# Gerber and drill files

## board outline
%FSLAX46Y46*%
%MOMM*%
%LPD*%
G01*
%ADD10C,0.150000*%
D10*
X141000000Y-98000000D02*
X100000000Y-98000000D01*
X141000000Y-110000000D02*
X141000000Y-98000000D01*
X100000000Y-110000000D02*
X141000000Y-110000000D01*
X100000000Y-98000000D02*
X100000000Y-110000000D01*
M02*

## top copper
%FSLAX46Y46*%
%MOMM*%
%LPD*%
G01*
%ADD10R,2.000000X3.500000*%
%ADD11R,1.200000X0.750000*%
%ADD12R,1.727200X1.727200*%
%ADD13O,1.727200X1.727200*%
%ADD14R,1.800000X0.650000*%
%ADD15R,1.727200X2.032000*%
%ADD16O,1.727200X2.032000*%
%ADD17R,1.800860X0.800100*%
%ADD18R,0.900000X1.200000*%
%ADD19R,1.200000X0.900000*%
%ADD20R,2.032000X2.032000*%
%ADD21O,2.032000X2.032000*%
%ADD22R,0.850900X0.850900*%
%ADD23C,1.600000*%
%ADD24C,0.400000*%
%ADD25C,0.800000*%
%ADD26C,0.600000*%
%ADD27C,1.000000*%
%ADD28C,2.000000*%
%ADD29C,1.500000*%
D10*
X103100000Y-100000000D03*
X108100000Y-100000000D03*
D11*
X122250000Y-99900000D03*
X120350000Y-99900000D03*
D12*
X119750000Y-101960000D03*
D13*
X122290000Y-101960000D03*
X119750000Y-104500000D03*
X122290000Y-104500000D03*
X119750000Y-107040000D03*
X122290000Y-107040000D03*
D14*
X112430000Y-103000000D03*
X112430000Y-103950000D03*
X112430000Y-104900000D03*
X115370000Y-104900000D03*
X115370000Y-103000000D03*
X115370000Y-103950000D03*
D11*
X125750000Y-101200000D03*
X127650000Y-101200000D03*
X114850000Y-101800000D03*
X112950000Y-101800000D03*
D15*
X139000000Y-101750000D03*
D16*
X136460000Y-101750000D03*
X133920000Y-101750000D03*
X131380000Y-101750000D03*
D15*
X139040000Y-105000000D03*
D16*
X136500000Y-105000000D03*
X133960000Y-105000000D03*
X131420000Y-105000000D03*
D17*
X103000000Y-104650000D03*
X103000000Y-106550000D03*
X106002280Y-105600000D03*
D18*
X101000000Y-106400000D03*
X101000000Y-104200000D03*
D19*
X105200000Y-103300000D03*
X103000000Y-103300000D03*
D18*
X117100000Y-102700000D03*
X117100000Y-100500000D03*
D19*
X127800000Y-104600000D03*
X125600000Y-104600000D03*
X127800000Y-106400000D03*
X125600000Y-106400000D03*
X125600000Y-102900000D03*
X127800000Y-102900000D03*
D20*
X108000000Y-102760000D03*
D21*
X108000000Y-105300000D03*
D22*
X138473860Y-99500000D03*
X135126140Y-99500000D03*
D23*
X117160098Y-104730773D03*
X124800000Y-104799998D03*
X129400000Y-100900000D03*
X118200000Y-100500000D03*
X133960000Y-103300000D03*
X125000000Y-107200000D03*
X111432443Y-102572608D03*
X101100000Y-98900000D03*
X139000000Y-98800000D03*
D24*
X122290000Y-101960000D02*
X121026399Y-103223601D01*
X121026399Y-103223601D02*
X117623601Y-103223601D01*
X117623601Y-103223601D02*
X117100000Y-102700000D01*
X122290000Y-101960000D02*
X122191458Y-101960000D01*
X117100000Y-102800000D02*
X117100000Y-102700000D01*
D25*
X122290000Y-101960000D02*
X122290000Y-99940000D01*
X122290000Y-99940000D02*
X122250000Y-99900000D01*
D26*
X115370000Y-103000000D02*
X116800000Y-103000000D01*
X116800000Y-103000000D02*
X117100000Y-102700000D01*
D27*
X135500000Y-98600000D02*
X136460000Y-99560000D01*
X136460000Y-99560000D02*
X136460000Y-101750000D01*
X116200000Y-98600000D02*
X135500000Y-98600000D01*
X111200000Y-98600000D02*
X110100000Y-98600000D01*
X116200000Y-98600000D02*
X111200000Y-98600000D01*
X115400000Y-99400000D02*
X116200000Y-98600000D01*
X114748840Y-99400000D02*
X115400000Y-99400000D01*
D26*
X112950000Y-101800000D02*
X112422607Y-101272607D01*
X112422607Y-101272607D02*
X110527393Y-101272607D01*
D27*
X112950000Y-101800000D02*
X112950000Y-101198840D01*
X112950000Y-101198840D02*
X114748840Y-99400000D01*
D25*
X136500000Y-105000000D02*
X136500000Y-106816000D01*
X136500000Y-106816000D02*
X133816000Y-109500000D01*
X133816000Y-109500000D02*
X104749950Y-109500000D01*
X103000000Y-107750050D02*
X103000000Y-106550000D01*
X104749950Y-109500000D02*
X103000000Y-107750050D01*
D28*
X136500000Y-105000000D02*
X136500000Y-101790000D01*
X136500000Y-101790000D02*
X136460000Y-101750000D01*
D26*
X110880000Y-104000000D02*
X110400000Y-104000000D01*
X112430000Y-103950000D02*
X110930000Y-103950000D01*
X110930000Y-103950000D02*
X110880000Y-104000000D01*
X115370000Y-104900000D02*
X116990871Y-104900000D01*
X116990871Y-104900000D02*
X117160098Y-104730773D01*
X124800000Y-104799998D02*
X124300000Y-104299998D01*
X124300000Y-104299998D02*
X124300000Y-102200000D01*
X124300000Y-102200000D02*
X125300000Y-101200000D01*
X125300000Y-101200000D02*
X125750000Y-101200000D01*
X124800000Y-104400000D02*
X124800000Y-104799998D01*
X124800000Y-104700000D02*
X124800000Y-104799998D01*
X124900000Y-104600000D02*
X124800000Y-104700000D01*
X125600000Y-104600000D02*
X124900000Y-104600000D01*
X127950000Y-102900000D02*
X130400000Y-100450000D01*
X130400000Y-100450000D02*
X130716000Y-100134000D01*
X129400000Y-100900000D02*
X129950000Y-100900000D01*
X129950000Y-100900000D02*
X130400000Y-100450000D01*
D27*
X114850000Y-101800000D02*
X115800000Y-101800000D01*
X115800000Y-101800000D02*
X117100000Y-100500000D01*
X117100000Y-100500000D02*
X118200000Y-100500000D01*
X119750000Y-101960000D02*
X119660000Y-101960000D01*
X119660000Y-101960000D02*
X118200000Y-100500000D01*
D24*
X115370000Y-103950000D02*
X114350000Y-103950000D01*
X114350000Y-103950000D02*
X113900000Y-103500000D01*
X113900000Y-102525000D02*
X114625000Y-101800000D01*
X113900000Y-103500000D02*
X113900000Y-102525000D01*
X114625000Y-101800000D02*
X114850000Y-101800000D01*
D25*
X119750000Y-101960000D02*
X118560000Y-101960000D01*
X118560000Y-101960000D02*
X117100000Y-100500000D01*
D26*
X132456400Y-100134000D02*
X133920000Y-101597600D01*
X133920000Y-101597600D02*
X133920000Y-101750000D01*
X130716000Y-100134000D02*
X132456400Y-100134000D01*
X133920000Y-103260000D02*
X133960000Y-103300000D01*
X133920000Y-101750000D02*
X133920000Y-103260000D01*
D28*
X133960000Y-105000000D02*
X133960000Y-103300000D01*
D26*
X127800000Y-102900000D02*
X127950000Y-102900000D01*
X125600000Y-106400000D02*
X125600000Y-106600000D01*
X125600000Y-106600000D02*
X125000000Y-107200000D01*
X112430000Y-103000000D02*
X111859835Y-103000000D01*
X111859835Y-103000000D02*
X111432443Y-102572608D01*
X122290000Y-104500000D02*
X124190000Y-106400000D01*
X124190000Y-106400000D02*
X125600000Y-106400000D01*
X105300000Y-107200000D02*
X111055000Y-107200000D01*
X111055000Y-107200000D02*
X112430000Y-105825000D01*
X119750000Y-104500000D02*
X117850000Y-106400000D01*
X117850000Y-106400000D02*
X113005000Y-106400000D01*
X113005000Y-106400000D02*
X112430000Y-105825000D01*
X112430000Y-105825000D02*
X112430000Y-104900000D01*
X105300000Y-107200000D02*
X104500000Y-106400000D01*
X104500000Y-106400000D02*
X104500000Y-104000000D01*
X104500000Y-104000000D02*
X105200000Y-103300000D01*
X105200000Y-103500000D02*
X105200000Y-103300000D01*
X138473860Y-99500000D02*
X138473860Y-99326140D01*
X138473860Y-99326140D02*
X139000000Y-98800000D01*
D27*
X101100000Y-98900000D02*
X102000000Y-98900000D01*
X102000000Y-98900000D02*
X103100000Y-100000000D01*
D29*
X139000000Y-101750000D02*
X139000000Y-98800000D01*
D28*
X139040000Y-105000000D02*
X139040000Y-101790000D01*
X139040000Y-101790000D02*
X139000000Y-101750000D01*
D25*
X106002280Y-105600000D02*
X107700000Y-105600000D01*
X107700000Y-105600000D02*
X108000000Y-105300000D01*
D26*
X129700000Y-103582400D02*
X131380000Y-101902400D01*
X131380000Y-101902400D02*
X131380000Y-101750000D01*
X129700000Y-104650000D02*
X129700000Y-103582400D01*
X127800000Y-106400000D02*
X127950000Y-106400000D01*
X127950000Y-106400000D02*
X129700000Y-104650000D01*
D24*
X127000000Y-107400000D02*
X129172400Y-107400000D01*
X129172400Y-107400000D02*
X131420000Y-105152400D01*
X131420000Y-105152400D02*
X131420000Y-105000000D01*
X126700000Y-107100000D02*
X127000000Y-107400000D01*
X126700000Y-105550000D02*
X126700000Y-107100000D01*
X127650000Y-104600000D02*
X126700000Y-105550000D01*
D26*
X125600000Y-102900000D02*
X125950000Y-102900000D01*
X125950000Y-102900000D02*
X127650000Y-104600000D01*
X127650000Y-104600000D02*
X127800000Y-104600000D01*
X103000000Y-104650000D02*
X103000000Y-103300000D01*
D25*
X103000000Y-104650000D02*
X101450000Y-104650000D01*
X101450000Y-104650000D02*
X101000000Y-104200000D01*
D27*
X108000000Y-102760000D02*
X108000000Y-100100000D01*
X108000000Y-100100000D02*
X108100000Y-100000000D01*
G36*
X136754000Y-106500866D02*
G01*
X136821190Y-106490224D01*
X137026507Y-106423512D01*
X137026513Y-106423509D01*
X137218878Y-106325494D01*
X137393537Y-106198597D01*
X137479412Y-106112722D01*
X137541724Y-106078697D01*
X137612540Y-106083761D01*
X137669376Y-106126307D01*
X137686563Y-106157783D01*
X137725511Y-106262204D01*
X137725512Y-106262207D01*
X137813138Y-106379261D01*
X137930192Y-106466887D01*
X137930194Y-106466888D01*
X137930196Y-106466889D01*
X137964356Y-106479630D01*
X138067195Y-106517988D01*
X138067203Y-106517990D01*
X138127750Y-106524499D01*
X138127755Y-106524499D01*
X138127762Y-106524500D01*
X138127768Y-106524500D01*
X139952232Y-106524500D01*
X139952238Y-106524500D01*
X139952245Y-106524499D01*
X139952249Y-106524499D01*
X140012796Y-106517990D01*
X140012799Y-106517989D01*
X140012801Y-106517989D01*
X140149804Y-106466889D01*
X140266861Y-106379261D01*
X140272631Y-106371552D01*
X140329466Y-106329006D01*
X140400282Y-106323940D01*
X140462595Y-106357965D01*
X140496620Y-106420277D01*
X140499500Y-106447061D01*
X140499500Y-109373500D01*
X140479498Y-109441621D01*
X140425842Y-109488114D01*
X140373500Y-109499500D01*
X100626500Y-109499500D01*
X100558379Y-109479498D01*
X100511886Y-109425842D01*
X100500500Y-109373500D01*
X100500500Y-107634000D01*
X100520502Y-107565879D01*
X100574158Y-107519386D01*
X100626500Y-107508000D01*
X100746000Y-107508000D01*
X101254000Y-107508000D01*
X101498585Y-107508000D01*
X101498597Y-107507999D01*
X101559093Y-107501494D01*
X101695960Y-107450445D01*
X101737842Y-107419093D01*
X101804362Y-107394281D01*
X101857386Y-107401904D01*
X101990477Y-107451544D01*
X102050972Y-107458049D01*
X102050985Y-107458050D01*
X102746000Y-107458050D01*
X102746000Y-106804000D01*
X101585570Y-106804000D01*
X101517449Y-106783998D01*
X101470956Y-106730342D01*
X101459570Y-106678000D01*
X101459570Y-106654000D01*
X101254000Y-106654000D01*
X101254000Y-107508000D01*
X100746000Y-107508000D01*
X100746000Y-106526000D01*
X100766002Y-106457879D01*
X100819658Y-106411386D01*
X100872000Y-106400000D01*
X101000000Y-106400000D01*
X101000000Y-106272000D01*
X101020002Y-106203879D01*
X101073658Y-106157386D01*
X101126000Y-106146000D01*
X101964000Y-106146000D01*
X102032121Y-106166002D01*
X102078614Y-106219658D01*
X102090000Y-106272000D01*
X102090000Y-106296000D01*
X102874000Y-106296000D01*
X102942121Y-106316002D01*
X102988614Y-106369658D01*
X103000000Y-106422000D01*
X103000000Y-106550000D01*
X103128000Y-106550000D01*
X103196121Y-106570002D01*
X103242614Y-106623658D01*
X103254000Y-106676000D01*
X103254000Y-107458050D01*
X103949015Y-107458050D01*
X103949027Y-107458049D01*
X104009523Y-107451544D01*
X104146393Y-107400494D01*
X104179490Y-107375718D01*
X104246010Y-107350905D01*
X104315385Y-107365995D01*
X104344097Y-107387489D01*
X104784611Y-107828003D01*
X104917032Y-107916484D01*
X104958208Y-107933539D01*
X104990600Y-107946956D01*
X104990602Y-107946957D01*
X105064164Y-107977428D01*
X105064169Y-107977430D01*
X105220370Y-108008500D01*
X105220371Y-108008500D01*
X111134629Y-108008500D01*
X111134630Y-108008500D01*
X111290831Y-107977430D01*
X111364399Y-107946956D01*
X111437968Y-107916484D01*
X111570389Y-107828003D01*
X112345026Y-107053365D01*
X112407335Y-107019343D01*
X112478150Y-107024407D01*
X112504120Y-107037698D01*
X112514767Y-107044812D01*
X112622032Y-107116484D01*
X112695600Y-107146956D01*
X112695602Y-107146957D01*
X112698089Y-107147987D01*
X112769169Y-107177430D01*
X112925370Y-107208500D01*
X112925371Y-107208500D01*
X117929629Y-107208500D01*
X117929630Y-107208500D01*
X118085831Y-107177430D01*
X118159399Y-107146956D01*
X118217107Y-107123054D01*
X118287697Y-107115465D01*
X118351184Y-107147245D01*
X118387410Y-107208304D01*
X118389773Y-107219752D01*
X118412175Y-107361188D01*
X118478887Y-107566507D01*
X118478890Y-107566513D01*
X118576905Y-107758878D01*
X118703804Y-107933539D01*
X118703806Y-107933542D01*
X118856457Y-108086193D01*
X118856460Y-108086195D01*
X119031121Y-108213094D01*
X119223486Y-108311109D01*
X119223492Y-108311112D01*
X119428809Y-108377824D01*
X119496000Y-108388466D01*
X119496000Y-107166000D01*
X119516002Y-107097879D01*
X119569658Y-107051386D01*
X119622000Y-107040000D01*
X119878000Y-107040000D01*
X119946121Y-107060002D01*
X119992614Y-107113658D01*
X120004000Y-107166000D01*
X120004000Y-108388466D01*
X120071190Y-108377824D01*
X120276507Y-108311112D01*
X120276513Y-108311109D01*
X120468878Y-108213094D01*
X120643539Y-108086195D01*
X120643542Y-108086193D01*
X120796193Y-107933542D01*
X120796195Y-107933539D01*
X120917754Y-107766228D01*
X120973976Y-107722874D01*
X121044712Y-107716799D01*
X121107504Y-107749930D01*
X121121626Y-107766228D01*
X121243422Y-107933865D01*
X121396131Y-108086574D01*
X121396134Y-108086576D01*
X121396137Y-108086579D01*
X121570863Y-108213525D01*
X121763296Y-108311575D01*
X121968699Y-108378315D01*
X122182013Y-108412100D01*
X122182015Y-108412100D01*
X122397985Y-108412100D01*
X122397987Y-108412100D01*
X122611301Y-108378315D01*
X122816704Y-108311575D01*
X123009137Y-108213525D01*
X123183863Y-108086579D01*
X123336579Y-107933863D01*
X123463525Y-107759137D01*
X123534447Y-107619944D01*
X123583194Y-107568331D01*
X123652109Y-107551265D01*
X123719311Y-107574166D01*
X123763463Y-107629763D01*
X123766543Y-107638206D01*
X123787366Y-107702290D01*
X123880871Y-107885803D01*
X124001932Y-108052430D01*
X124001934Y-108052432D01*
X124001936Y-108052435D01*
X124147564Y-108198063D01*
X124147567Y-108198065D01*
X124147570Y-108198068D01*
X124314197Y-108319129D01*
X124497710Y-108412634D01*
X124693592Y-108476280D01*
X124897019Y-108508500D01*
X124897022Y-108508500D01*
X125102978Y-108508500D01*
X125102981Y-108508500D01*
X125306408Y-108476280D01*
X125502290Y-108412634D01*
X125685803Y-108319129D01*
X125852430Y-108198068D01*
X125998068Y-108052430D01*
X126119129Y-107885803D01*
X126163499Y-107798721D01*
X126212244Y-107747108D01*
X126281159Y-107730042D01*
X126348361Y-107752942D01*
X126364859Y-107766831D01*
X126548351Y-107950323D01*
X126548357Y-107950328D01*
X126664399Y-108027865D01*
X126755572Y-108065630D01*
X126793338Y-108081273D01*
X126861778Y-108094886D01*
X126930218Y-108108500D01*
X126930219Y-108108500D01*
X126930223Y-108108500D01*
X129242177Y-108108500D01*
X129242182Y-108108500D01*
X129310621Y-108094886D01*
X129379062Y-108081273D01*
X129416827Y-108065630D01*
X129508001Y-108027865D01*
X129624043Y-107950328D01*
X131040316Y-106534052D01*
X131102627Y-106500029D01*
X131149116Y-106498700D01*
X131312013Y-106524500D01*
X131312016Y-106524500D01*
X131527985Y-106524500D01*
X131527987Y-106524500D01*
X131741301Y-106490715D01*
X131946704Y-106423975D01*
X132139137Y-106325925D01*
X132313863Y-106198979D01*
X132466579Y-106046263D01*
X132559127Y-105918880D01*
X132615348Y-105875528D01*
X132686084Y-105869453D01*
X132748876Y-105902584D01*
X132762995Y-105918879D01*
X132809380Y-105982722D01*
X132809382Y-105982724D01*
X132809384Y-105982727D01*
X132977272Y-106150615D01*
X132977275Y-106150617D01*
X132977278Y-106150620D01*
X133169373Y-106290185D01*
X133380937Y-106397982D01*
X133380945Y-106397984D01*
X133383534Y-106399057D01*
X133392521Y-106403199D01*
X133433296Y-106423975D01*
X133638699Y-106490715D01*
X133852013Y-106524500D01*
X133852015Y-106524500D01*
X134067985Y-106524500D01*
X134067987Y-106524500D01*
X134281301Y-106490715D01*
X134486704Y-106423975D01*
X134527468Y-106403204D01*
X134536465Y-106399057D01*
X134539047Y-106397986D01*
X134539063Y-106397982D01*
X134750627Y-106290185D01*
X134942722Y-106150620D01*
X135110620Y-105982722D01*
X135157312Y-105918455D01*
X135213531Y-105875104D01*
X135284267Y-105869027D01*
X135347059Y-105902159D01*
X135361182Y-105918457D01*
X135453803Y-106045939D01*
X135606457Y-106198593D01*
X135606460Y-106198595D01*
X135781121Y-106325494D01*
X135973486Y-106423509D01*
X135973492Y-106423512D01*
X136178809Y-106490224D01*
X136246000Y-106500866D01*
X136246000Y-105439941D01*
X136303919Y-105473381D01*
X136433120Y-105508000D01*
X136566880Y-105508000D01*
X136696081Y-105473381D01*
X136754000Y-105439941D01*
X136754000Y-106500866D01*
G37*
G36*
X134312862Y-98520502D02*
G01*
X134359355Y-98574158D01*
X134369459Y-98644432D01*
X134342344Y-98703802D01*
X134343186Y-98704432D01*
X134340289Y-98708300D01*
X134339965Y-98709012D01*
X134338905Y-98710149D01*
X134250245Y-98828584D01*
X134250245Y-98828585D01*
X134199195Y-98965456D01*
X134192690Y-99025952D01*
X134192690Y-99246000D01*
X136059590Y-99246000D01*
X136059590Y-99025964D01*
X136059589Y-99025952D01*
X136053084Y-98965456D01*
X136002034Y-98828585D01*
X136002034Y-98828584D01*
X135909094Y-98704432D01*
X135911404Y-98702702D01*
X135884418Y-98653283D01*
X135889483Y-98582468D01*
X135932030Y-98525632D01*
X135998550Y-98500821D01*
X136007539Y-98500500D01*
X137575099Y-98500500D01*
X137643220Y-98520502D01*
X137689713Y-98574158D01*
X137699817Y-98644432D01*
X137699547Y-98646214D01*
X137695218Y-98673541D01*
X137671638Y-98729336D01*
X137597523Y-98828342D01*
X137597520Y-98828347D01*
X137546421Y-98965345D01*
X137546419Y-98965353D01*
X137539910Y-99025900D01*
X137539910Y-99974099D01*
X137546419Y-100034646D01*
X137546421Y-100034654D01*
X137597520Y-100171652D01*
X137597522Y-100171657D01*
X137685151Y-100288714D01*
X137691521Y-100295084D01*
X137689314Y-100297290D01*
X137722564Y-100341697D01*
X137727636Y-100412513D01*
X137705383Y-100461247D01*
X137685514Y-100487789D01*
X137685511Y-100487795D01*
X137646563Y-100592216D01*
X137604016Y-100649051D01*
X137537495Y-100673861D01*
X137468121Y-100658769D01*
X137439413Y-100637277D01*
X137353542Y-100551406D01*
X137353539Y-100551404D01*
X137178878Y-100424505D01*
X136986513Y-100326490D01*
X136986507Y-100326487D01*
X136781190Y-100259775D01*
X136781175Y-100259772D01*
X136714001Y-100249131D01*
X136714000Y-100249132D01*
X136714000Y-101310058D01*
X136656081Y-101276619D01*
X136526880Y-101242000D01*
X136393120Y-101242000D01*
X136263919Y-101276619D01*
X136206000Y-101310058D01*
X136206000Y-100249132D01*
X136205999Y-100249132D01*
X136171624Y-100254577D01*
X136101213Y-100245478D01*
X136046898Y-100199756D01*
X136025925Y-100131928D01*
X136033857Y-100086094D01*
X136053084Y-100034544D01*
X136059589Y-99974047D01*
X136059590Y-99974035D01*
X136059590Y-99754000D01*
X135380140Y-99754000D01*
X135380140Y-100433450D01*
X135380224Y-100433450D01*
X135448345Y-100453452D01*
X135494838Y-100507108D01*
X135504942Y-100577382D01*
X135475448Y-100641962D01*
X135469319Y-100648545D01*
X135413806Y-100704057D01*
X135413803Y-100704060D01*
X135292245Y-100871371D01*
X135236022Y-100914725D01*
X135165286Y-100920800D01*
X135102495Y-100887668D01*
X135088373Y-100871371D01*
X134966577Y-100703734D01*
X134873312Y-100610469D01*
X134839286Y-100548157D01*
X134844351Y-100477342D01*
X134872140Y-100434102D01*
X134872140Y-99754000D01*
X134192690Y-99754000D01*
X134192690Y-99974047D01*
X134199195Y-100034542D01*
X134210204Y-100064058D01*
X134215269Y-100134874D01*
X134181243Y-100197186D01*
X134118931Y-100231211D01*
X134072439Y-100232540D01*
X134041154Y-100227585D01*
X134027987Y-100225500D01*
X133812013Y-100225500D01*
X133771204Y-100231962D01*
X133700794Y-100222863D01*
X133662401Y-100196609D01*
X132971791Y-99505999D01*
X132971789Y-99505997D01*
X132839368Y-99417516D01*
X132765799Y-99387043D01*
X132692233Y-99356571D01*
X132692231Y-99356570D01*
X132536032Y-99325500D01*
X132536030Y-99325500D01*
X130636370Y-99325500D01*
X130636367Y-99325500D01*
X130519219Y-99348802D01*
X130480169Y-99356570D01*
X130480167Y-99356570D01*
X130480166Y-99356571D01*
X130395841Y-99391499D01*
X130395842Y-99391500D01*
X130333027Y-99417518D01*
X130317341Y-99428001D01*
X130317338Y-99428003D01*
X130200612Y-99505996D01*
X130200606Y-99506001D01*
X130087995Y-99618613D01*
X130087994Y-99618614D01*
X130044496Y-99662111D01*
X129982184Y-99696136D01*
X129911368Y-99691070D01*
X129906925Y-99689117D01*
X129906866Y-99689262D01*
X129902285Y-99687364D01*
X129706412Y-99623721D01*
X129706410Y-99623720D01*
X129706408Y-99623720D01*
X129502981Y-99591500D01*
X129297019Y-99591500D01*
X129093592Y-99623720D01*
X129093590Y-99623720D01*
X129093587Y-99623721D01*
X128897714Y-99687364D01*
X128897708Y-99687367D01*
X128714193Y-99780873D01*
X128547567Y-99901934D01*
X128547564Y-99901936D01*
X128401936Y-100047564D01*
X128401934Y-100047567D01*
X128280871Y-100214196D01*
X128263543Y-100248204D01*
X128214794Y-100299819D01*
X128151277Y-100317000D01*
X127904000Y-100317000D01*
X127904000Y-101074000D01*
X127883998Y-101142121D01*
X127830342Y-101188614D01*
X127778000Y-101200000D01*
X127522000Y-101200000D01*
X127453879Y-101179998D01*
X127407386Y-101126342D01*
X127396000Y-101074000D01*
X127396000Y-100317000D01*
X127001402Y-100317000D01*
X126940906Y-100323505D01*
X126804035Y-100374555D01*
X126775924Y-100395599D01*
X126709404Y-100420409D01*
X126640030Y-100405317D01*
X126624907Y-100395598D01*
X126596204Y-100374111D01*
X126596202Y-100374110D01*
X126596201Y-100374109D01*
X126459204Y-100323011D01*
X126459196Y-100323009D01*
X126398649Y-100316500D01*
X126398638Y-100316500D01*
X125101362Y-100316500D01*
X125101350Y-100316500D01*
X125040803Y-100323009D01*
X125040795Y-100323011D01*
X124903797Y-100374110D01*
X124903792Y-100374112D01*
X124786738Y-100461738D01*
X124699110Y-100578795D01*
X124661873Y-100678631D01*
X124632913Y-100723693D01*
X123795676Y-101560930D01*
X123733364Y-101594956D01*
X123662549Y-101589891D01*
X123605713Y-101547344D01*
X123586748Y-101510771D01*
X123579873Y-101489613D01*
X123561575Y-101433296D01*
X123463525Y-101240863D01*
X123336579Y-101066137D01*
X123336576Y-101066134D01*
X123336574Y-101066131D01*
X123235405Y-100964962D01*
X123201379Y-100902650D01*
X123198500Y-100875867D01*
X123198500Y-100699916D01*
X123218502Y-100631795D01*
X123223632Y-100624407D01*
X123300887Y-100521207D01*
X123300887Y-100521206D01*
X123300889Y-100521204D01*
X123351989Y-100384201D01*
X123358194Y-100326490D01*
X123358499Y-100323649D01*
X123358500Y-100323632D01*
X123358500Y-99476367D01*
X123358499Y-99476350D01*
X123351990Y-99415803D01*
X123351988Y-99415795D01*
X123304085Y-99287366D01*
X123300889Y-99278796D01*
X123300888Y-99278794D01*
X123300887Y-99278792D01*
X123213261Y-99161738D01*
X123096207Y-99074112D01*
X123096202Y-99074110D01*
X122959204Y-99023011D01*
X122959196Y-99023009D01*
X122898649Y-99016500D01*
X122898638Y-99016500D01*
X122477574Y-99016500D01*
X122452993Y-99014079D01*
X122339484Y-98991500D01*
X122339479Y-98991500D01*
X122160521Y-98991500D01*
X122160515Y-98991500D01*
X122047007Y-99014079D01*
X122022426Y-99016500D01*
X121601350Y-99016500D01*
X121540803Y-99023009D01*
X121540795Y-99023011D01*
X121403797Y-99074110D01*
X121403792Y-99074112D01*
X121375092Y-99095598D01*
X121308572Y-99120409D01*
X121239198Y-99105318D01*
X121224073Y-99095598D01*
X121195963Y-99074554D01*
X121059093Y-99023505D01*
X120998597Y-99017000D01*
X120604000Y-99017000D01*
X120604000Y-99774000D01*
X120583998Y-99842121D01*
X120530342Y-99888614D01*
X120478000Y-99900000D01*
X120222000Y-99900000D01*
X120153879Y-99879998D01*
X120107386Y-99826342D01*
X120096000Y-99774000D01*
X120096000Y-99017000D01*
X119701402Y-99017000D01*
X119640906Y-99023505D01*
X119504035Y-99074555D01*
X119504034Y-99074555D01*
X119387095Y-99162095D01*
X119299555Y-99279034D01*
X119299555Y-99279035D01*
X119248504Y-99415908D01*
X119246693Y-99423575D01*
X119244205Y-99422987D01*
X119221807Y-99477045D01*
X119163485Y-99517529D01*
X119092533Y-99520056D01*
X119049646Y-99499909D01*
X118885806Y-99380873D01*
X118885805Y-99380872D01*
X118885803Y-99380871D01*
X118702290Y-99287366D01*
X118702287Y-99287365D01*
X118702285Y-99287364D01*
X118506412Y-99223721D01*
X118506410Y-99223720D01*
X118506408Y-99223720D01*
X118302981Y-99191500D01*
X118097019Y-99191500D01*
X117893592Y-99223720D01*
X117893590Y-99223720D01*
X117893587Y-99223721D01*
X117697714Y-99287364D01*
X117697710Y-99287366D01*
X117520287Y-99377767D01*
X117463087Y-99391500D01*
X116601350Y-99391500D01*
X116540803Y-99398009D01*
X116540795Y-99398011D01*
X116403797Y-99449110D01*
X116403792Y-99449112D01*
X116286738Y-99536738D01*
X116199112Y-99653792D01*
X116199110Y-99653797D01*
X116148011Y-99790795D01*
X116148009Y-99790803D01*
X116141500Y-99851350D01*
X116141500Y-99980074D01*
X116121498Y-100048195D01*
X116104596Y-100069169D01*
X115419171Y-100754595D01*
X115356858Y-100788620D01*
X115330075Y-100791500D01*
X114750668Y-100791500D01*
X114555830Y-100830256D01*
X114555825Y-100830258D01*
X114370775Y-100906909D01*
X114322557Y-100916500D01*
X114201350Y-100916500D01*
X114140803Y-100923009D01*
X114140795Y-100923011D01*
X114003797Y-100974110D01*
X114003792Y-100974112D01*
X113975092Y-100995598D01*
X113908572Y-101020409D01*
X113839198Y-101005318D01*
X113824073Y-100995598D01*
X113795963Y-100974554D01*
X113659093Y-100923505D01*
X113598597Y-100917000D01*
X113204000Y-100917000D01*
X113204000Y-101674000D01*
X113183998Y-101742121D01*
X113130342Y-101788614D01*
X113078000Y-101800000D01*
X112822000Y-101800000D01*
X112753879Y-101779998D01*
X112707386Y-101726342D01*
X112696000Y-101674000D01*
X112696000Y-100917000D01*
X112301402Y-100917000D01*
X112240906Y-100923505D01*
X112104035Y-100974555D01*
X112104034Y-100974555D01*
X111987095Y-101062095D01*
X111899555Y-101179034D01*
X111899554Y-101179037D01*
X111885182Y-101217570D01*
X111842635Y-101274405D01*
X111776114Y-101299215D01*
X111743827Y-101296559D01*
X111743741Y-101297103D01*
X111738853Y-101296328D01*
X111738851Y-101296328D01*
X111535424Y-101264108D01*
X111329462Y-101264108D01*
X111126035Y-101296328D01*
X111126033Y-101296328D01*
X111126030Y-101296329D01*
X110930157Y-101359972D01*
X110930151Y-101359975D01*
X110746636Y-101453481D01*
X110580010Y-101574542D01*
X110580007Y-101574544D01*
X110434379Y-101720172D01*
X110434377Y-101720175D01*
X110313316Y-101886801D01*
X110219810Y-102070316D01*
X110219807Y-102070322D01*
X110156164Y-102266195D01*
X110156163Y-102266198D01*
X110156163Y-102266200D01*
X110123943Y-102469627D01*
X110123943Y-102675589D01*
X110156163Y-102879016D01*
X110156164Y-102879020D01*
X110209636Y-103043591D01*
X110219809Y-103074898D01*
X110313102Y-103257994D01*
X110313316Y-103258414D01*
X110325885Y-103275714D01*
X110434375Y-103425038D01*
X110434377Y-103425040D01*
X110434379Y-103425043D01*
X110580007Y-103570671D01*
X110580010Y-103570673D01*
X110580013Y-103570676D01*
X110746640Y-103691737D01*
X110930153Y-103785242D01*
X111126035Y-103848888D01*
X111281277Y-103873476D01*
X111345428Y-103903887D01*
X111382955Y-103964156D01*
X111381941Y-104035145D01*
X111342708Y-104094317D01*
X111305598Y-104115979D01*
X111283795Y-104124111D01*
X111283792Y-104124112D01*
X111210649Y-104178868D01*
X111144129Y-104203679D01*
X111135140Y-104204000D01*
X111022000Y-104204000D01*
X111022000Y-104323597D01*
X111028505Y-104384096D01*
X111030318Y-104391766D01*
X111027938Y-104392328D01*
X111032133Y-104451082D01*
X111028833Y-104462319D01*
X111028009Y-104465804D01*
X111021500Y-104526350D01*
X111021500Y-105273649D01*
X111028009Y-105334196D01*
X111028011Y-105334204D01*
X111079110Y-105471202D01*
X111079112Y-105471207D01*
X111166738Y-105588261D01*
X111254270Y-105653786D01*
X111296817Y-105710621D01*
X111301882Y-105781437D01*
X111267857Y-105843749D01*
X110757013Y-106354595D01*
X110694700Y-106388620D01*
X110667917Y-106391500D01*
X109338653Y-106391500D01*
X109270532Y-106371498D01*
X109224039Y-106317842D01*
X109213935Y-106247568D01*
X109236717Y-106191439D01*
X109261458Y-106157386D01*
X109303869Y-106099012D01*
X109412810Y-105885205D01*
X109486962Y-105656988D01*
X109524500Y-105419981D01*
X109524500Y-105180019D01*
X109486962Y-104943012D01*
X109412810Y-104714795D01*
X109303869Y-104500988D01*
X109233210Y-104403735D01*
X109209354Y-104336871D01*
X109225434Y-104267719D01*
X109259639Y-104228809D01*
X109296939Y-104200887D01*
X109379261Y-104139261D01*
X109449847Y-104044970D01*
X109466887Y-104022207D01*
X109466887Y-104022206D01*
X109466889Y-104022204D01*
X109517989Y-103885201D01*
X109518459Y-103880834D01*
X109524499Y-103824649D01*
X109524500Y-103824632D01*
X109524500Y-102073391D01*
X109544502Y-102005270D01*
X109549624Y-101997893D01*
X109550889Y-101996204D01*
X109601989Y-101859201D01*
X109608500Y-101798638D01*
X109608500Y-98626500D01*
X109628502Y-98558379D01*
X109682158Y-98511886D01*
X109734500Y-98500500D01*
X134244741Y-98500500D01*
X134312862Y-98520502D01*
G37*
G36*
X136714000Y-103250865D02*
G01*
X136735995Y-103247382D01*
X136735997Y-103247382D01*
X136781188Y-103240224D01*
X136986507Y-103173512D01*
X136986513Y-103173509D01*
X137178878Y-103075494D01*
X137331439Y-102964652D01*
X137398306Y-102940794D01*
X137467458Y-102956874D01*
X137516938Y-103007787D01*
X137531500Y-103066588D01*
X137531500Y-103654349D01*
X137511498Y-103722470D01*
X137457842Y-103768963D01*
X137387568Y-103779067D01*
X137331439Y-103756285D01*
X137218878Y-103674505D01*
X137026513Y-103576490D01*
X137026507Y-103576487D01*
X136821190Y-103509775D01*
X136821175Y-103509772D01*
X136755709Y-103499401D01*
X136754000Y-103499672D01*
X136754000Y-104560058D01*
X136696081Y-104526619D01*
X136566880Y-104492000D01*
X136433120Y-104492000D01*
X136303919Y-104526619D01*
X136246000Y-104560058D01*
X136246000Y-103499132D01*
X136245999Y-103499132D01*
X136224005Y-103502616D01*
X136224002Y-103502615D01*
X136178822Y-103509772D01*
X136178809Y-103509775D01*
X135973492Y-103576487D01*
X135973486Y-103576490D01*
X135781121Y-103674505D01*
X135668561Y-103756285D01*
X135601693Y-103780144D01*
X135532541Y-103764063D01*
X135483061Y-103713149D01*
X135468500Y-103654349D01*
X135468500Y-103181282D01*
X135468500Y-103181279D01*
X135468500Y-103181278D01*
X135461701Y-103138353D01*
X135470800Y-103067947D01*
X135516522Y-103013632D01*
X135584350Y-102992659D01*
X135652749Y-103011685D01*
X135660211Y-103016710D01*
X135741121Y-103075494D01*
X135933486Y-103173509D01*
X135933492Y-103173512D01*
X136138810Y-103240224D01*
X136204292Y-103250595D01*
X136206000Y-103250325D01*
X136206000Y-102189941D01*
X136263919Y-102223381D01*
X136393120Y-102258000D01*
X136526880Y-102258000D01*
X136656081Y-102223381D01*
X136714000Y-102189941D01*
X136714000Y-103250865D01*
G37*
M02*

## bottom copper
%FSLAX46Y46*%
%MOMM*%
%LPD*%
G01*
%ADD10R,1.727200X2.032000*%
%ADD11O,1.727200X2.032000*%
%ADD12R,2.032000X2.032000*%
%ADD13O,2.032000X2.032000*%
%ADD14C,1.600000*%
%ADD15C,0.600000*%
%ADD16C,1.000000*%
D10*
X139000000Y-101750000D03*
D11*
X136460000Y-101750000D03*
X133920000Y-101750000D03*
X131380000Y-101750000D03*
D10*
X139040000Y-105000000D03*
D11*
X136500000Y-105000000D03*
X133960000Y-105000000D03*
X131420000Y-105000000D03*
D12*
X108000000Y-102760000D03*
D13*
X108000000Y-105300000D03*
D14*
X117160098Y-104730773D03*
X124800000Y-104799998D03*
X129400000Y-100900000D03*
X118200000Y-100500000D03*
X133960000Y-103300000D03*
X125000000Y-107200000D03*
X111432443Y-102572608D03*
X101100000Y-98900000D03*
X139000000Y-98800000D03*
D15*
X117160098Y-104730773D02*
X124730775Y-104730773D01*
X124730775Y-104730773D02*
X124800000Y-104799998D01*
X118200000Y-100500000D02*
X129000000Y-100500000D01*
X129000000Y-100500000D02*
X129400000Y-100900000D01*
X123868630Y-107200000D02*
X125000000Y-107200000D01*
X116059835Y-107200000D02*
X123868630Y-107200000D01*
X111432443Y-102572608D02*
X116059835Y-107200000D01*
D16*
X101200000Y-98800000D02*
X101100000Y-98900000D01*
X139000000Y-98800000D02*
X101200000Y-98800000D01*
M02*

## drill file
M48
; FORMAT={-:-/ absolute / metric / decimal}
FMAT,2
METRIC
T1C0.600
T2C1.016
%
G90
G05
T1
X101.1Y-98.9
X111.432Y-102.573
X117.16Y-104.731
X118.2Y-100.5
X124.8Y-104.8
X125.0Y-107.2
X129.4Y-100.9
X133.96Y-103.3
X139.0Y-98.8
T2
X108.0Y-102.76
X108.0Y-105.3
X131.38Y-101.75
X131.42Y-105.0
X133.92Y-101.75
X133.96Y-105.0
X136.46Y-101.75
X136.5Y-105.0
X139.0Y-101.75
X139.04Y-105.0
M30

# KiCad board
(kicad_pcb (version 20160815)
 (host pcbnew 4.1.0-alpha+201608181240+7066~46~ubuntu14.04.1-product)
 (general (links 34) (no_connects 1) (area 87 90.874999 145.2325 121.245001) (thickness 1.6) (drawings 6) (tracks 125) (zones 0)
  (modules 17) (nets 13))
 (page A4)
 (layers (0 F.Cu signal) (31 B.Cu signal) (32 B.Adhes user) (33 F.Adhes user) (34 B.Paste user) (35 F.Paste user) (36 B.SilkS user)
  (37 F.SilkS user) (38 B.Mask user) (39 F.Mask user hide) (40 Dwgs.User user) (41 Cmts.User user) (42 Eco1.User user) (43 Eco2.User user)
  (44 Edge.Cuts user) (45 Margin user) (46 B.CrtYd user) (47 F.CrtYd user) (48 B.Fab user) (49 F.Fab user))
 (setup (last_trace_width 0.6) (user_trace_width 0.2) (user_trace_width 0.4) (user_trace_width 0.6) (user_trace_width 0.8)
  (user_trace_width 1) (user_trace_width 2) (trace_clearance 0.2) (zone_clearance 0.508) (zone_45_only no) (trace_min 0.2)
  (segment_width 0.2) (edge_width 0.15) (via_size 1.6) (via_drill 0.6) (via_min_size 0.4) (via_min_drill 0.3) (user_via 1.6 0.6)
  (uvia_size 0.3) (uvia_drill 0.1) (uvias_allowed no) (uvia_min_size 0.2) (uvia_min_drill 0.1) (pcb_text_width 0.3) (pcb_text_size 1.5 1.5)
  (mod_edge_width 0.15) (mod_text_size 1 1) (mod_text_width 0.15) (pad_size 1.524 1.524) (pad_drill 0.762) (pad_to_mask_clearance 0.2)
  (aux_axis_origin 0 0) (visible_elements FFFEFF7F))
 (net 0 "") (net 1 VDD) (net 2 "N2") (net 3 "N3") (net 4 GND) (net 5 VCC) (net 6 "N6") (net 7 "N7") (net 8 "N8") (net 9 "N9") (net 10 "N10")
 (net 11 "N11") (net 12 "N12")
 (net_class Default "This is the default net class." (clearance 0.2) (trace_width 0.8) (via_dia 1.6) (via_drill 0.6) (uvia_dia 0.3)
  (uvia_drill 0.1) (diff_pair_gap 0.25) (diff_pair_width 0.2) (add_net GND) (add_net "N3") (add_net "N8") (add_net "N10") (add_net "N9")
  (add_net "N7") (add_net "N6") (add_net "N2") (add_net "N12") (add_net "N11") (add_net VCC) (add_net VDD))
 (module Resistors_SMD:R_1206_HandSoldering (layer F.Cu) (at 105.6 100)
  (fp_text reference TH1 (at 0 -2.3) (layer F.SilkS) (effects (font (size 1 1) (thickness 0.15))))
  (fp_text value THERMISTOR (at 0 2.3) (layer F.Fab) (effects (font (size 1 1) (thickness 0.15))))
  (pad 1 smd rect (at -2.5 0) (size 2 3.5) (layers F.Cu F.Paste F.Mask) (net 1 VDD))
  (pad 2 smd rect (at 2.5 0) (size 2 3.5) (layers F.Cu F.Paste F.Mask) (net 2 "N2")))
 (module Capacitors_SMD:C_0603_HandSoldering (layer F.Cu) (at 121.3 99.9 180)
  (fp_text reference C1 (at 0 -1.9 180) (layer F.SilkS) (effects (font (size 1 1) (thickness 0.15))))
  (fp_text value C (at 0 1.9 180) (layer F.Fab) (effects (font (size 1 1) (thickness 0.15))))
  (pad 1 smd rect (at -0.95 0 180) (size 1.2 0.75) (layers F.Cu F.Paste F.Mask) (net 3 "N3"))
  (pad 2 smd rect (at 0.95 0 180) (size 1.2 0.75) (layers F.Cu F.Paste F.Mask) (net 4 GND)))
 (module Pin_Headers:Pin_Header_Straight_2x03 (layer F.Cu) (at 119.75 101.96)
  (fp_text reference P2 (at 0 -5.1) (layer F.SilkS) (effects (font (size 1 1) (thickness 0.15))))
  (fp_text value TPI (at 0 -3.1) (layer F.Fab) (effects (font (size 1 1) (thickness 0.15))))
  (pad 1 smd rect (at 0 0) (size 1.7272 1.7272) (layers F.Cu F.Paste F.Mask) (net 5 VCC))
  (pad 2 smd oval (at 2.54 0) (size 1.7272 1.7272) (layers F.Cu F.Paste F.Mask) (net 3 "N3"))
  (pad 3 smd oval (at 0 2.54) (size 1.7272 1.7272) (layers F.Cu F.Paste F.Mask) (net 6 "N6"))
  (pad 4 smd oval (at 2.54 2.54) (size 1.7272 1.7272) (layers F.Cu F.Paste F.Mask) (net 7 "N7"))
  (pad 5 smd oval (at 0 5.08) (size 1.7272 1.7272) (layers F.Cu F.Paste F.Mask) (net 4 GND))
  (pad 6 smd oval (at 2.54 5.08) (size 1.7272 1.7272) (layers F.Cu F.Paste F.Mask)))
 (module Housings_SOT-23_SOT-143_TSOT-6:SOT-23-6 (layer F.Cu) (at 113.9 103.95)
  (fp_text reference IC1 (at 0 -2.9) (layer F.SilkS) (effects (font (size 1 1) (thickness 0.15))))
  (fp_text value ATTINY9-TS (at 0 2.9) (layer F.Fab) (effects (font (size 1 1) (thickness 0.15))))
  (pad 1 smd rect (at -1.47 -0.95) (size 1.8 0.65) (layers F.Cu F.Paste F.Mask) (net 7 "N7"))
  (pad 2 smd rect (at -1.47 0) (size 1.8 0.65) (layers F.Cu F.Paste F.Mask) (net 4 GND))
  (pad 3 smd rect (at -1.47 0.95) (size 1.8 0.65) (layers F.Cu F.Paste F.Mask) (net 6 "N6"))
  (pad 4 smd rect (at 1.47 0.95) (size 1.8 0.65) (layers F.Cu F.Paste F.Mask) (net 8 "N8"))
  (pad 6 smd rect (at 1.47 -0.95) (size 1.8 0.65) (layers F.Cu F.Paste F.Mask) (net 3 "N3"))
  (pad 5 smd rect (at 1.47 0) (size 1.8 0.65) (layers F.Cu F.Paste F.Mask) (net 5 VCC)))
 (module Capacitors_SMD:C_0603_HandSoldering (layer F.Cu) (at 126.7 101.2)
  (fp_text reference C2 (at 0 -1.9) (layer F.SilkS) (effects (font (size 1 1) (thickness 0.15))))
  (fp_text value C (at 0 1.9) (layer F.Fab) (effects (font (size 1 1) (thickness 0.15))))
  (pad 1 smd rect (at -0.95 0) (size 1.2 0.75) (layers F.Cu F.Paste F.Mask) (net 8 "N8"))
  (pad 2 smd rect (at 0.95 0) (size 1.2 0.75) (layers F.Cu F.Paste F.Mask) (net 4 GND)))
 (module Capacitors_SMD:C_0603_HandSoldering (layer F.Cu) (at 113.9 101.8 180)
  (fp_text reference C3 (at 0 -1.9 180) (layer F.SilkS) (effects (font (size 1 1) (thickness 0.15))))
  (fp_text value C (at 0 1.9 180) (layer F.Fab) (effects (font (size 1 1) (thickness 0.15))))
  (pad 1 smd rect (at -0.95 0 180) (size 1.2 0.75) (layers F.Cu F.Paste F.Mask) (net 5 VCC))
  (pad 2 smd rect (at 0.95 0 180) (size 1.2 0.75) (layers F.Cu F.Paste F.Mask) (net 4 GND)))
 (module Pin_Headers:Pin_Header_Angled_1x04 (layer B.Cu) (at 139 101.75 90)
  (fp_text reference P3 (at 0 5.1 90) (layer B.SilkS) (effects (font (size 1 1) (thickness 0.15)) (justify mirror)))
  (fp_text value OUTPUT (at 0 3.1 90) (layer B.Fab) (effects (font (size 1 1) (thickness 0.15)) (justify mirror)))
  (pad 1 thru_hole rect (at 0 0 90) (size 2.032 1.7272) (drill 1.016) (layers *.Cu *.Mask B.SilkS) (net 1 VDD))
  (pad 2 thru_hole oval (at 0 -2.54 90) (size 2.032 1.7272) (drill 1.016) (layers *.Cu *.Mask B.SilkS) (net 4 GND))
  (pad 3 thru_hole oval (at 0 -5.08 90) (size 2.032 1.7272) (drill 1.016) (layers *.Cu *.Mask B.SilkS) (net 5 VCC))
  (pad 4 thru_hole oval (at 0 -7.62 90) (size 2.032 1.7272) (drill 1.016) (layers *.Cu *.Mask B.SilkS) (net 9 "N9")))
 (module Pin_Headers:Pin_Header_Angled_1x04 (layer F.Cu) (at 139.04 105 270)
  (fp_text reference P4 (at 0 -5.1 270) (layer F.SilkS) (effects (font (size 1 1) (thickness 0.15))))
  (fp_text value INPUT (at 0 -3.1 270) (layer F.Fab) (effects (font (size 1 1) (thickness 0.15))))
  (pad 1 thru_hole rect (at 0 0 270) (size 2.032 1.7272) (drill 1.016) (layers *.Cu *.Mask F.SilkS) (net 1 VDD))
  (pad 2 thru_hole oval (at 0 2.54 270) (size 2.032 1.7272) (drill 1.016) (layers *.Cu *.Mask F.SilkS) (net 4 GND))
  (pad 3 thru_hole oval (at 0 5.08 270) (size 2.032 1.7272) (drill 1.016) (layers *.Cu *.Mask F.SilkS) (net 5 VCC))
  (pad 4 thru_hole oval (at 0 7.62 270) (size 2.032 1.7272) (drill 1.016) (layers *.Cu *.Mask F.SilkS) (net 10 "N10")))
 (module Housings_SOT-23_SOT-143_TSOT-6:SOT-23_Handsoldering (layer F.Cu) (at 104.50114 105.6 270)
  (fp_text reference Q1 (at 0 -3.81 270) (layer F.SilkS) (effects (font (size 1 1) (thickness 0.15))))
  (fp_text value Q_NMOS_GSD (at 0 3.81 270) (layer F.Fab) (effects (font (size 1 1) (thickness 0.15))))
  (pad 1 smd rect (at -0.95 1.50114 270) (size 0.8001 1.80086) (layers F.Cu F.Paste F.Mask) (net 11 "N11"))
  (pad 2 smd rect (at 0.95 1.50114 270) (size 0.8001 1.80086) (layers F.Cu F.Paste F.Mask) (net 4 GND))
  (pad 3 smd rect (at 0 -1.50114 270) (size 0.8001 1.80086) (layers F.Cu F.Paste F.Mask) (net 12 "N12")))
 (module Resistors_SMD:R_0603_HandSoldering (layer F.Cu) (at 101 105.3 90)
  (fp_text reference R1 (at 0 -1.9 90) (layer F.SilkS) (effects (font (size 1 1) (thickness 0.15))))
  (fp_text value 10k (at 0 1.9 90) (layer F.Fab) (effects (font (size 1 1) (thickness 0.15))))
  (pad 1 smd rect (at -1.1 0 90) (size 1.2 0.9) (layers F.Cu F.Paste F.Mask) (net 4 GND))
  (pad 2 smd rect (at 1.1 0 90) (size 1.2 0.9) (layers F.Cu F.Paste F.Mask) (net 11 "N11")))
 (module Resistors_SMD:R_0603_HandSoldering (layer F.Cu) (at 104.1 103.3 180)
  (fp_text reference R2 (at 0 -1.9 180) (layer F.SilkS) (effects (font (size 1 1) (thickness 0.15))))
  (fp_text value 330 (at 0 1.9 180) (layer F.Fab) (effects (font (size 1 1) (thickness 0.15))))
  (pad 1 smd rect (at -1.1 0 180) (size 1.2 0.9) (layers F.Cu F.Paste F.Mask) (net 6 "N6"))
  (pad 2 smd rect (at 1.1 0 180) (size 1.2 0.9) (layers F.Cu F.Paste F.Mask) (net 11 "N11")))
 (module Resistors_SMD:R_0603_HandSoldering (layer F.Cu) (at 117.1 101.6 90)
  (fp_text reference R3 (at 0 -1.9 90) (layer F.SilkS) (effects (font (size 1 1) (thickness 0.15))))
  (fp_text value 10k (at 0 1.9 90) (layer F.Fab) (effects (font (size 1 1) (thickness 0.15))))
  (pad 1 smd rect (at -1.1 0 90) (size 1.2 0.9) (layers F.Cu F.Paste F.Mask) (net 3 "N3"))
  (pad 2 smd rect (at 1.1 0 90) (size 1.2 0.9) (layers F.Cu F.Paste F.Mask) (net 5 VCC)))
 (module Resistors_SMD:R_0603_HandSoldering (layer F.Cu) (at 126.7 104.6 180)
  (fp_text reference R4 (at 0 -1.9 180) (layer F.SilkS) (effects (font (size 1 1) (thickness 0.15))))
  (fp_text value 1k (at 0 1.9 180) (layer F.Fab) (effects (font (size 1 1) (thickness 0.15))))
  (pad 1 smd rect (at -1.1 0 180) (size 1.2 0.9) (layers F.Cu F.Paste F.Mask) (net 10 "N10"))
  (pad 2 smd rect (at 1.1 0 180) (size 1.2 0.9) (layers F.Cu F.Paste F.Mask) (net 8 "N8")))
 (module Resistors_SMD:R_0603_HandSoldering (layer F.Cu) (at 126.7 106.4 180)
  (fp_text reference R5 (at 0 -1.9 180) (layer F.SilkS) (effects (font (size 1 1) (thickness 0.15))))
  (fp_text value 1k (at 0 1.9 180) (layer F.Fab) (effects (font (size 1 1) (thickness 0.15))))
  (pad 1 smd rect (at -1.1 0 180) (size 1.2 0.9) (layers F.Cu F.Paste F.Mask) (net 9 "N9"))
  (pad 2 smd rect (at 1.1 0 180) (size 1.2 0.9) (layers F.Cu F.Paste F.Mask) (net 7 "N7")))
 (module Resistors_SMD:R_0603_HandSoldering (layer F.Cu) (at 126.7 102.9)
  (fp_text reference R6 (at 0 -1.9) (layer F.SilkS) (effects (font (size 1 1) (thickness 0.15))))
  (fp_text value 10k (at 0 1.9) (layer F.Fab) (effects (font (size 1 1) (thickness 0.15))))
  (pad 1 smd rect (at -1.1 0) (size 1.2 0.9) (layers F.Cu F.Paste F.Mask) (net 10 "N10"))
  (pad 2 smd rect (at 1.1 0) (size 1.2 0.9) (layers F.Cu F.Paste F.Mask) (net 5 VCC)))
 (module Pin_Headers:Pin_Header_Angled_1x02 (layer B.Cu) (at 108 102.76 180)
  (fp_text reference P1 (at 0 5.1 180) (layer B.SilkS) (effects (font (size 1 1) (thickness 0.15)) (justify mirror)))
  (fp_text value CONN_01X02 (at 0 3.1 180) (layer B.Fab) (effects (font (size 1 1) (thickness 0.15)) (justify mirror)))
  (pad 1 thru_hole rect (at 0 0 180) (size 2.032 2.032) (drill 1.016) (layers *.Cu *.Mask B.SilkS) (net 2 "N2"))
  (pad 2 thru_hole oval (at 0 -2.54 180) (size 2.032 2.032) (drill 1.016) (layers *.Cu *.Mask B.SilkS) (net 12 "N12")))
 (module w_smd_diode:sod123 (layer F.Cu) (at 136.8 99.5)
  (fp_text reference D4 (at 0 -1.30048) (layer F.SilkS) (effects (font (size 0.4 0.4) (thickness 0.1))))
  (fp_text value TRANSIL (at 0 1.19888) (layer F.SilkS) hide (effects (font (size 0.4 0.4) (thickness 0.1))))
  (pad 2 smd rect (at 1.67386 0) (size 0.8509 0.8509) (layers F.Cu F.Paste F.Mask) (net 1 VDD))
  (pad 1 smd rect (at -1.67386 0) (size 0.8509 0.8509) (layers F.Cu F.Paste F.Mask) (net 4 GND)))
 (gr_line (start 141 98) (end 100 98) (layer Edge.Cuts) (width 0.15))
 (gr_line (start 141 110) (end 141 98) (layer Edge.Cuts) (width 0.15))
 (gr_line (start 100 110) (end 141 110) (layer Edge.Cuts) (width 0.15))
 (gr_line (start 100 98) (end 100 110) (layer Edge.Cuts) (width 0.15))
 (segment (start 122.29 101.96) (end 121.026399 103.223601) (width 0.4) (layer F.Cu) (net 3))
 (segment (start 121.026399 103.223601) (end 117.623601 103.223601) (width 0.4) (layer F.Cu) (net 3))
 (segment (start 117.623601 103.223601) (end 117.1 102.7) (width 0.4) (layer F.Cu) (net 3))
 (segment (start 122.29 101.96) (end 122.191458 101.96) (width 0.4) (layer F.Cu) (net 3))
 (segment (start 117.1 102.8) (end 117.1 102.7) (width 0.4) (layer F.Cu) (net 3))
 (segment (start 122.29 101.96) (end 122.29 99.94) (width 0.8) (layer F.Cu) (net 3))
 (segment (start 122.29 99.94) (end 122.25 99.9) (width 0.8) (layer F.Cu) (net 3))
 (segment (start 115.37 103) (end 116.8 103) (width 0.6) (layer F.Cu) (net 3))
 (segment (start 116.8 103) (end 117.1 102.7) (width 0.6) (layer F.Cu) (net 3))
 (segment (start 135.5 98.6) (end 136.46 99.56) (width 1) (layer F.Cu) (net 4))
 (segment (start 136.46 99.56) (end 136.46 101.75) (width 1) (layer F.Cu) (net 4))
 (segment (start 116.2 98.6) (end 135.5 98.6) (width 1) (layer F.Cu) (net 4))
 (segment (start 111.2 98.6) (end 110.1 98.6) (width 1) (layer F.Cu) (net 4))
 (segment (start 116.2 98.6) (end 111.2 98.6) (width 1) (layer F.Cu) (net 4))
 (segment (start 115.4 99.4) (end 116.2 98.6) (width 1) (layer F.Cu) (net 4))
 (segment (start 114.74884 99.4) (end 115.4 99.4) (width 1) (layer F.Cu) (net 4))
 (segment (start 112.95 101.8) (end 112.422607 101.272607) (width 0.6) (layer F.Cu) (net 4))
 (segment (start 112.422607 101.272607) (end 110.527393 101.272607) (width 0.6) (layer F.Cu) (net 4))
 (segment (start 112.95 101.8) (end 112.95 101.19884) (width 1) (layer F.Cu) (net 4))
 (segment (start 112.95 101.19884) (end 114.74884 99.4) (width 1) (layer F.Cu) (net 4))
 (segment (start 136.5 105) (end 136.5 106.816) (width 0.8) (layer F.Cu) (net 4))
 (segment (start 136.5 106.816) (end 133.816 109.5) (width 0.8) (layer F.Cu) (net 4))
 (segment (start 133.816 109.5) (end 104.74995 109.5) (width 0.8) (layer F.Cu) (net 4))
 (segment (start 103 107.75005) (end 103 106.55) (width 0.8) (layer F.Cu) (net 4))
 (segment (start 104.74995 109.5) (end 103 107.75005) (width 0.8) (layer F.Cu) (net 4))
 (segment (start 136.5 105) (end 136.5 101.79) (width 2) (layer F.Cu) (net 4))
 (segment (start 136.5 101.79) (end 136.46 101.75) (width 2) (layer F.Cu) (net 4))
 (segment (start 110.88 104) (end 110.4 104) (width 0.6) (layer F.Cu) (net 4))
 (segment (start 112.43 103.95) (end 110.93 103.95) (width 0.6) (layer F.Cu) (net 4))
 (segment (start 110.93 103.95) (end 110.88 104) (width 0.6) (layer F.Cu) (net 4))
 (segment (start 117.160098 104.730773) (end 124.730775 104.730773) (width 0.6) (layer B.Cu) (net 8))
 (segment (start 124.730775 104.730773) (end 124.8 104.799998) (width 0.6) (layer B.Cu) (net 8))
 (segment (start 115.37 104.9) (end 116.990871 104.9) (width 0.6) (layer F.Cu) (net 8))
 (segment (start 116.990871 104.9) (end 117.160098 104.730773) (width 0.6) (layer F.Cu) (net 8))
 (via (at 117.160098 104.730773) (size 1.6) (drill 0.6) (layers F.Cu B.Cu) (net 8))
 (segment (start 124.8 104.799998) (end 124.3 104.299998) (width 0.6) (layer F.Cu) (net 8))
 (segment (start 124.3 104.299998) (end 124.3 102.2) (width 0.6) (layer F.Cu) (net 8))
 (segment (start 124.3 102.2) (end 125.3 101.2) (width 0.6) (layer F.Cu) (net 8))
 (segment (start 125.3 101.2) (end 125.75 101.2) (width 0.6) (layer F.Cu) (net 8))
 (segment (start 124.8 104.4) (end 124.8 104.799998) (width 0.6) (layer F.Cu) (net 8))
 (segment (start 124.8 104.7) (end 124.8 104.799998) (width 0.6) (layer F.Cu) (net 8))
 (segment (start 124.9 104.6) (end 124.8 104.7) (width 0.6) (layer F.Cu) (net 8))
 (segment (start 125.6 104.6) (end 124.9 104.6) (width 0.6) (layer F.Cu) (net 8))
 (via (at 124.8 104.799998) (size 1.6) (drill 0.6) (layers F.Cu B.Cu) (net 8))
 (segment (start 127.95 102.9) (end 130.4 100.45) (width 0.6) (layer F.Cu) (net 5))
 (segment (start 130.4 100.45) (end 130.716 100.134) (width 0.6) (layer F.Cu) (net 5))
 (segment (start 129.4 100.9) (end 129.95 100.9) (width 0.6) (layer F.Cu) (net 5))
 (segment (start 129.95 100.9) (end 130.4 100.45) (width 0.6) (layer F.Cu) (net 5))
 (segment (start 114.85 101.8) (end 115.8 101.8) (width 1) (layer F.Cu) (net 5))
 (segment (start 115.8 101.8) (end 117.1 100.5) (width 1) (layer F.Cu) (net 5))
 (segment (start 117.1 100.5) (end 118.2 100.5) (width 1) (layer F.Cu) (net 5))
 (segment (start 119.75 101.96) (end 119.66 101.96) (width 1) (layer F.Cu) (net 5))
 (segment (start 119.66 101.96) (end 118.2 100.5) (width 1) (layer F.Cu) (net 5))
 (segment (start 118.2 100.5) (end 129 100.5) (width 0.6) (layer B.Cu) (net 5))
 (segment (start 129 100.5) (end 129.4 100.9) (width 0.6) (layer B.Cu) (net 5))
 (via (at 129.4 100.9) (size 1.6) (drill 0.6) (layers F.Cu B.Cu) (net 5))
 (via (at 118.2 100.5) (size 1.6) (drill 0.6) (layers F.Cu B.Cu) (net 5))
 (segment (start 115.37 103.95) (end 114.35 103.95) (width 0.4) (layer F.Cu) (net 5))
 (segment (start 114.35 103.95) (end 113.9 103.5) (width 0.4) (layer F.Cu) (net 5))
 (segment (start 113.9 102.525) (end 114.625 101.8) (width 0.4) (layer F.Cu) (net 5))
 (segment (start 113.9 103.5) (end 113.9 102.525) (width 0.4) (layer F.Cu) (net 5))
 (segment (start 114.625 101.8) (end 114.85 101.8) (width 0.4) (layer F.Cu) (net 5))
 (segment (start 119.75 101.96) (end 118.56 101.96) (width 0.8) (layer F.Cu) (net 5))
 (segment (start 118.56 101.96) (end 117.1 100.5) (width 0.8) (layer F.Cu) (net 5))
 (segment (start 132.4564 100.134) (end 133.92 101.5976) (width 0.6) (layer F.Cu) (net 5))
 (segment (start 133.92 101.5976) (end 133.92 101.75) (width 0.6) (layer F.Cu) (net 5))
 (segment (start 130.716 100.134) (end 132.4564 100.134) (width 0.6) (layer F.Cu) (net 5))
 (segment (start 133.92 103.26) (end 133.96 103.3) (width 0.6) (layer F.Cu) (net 5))
 (segment (start 133.92 101.75) (end 133.92 103.26) (width 0.6) (layer F.Cu) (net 5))
 (via (at 133.96 103.3) (size 1.6) (drill 0.6) (layers F.Cu B.Cu) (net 5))
 (segment (start 133.96 105) (end 133.96 103.3) (width 2) (layer F.Cu) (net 5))
 (segment (start 127.8 102.9) (end 127.95 102.9) (width 0.6) (layer F.Cu) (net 5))
 (segment (start 123.86863 107.2) (end 125 107.2) (width 0.6) (layer B.Cu) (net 7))
 (segment (start 116.059835 107.2) (end 123.86863 107.2) (width 0.6) (layer B.Cu) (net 7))
 (segment (start 111.432443 102.572608) (end 116.059835 107.2) (width 0.6) (layer B.Cu) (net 7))
 (segment (start 125.6 106.4) (end 125.6 106.6) (width 0.6) (layer F.Cu) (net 7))
 (segment (start 125.6 106.6) (end 125 107.2) (width 0.6) (layer F.Cu) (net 7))
 (via (at 125 107.2) (size 1.6) (drill 0.6) (layers F.Cu B.Cu) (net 7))
 (segment (start 112.43 103) (end 111.859835 103) (width 0.6) (layer F.Cu) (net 7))
 (segment (start 111.859835 103) (end 111.432443 102.572608) (width 0.6) (layer F.Cu) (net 7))
 (via (at 111.432443 102.572608) (size 1.6) (drill 0.6) (layers F.Cu B.Cu) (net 7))
 (segment (start 122.29 104.5) (end 124.19 106.4) (width 0.6) (layer F.Cu) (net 7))
 (segment (start 124.19 106.4) (end 125.6 106.4) (width 0.6) (layer F.Cu) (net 7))
 (segment (start 105.3 107.2) (end 111.055 107.2) (width 0.6) (layer F.Cu) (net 6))
 (segment (start 111.055 107.2) (end 112.43 105.825) (width 0.6) (layer F.Cu) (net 6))
 (segment (start 119.75 104.5) (end 117.85 106.4) (width 0.6) (layer F.Cu) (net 6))
 (segment (start 117.85 106.4) (end 113.005 106.4) (width 0.6) (layer F.Cu) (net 6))
 (segment (start 113.005 106.4) (end 112.43 105.825) (width 0.6) (layer F.Cu) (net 6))
 (segment (start 112.43 105.825) (end 112.43 104.9) (width 0.6) (layer F.Cu) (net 6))
 (segment (start 105.3 107.2) (end 104.5 106.4) (width 0.6) (layer F.Cu) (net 6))
 (segment (start 104.5 106.4) (end 104.5 104) (width 0.6) (layer F.Cu) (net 6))
 (segment (start 104.5 104) (end 105.2 103.3) (width 0.6) (layer F.Cu) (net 6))
 (segment (start 105.2 103.5) (end 105.2 103.3) (width 0.6) (layer F.Cu) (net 6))
 (segment (start 138.47386 99.5) (end 138.47386 99.32614) (width 0.6) (layer F.Cu) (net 1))
 (segment (start 138.47386 99.32614) (end 139 98.8) (width 0.6) (layer F.Cu) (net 1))
 (segment (start 101.1 98.9) (end 102 98.9) (width 1) (layer F.Cu) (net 1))
 (segment (start 102 98.9) (end 103.1 100) (width 1) (layer F.Cu) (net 1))
 (segment (start 101.2 98.8) (end 101.1 98.9) (width 1) (layer B.Cu) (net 1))
 (segment (start 139 98.8) (end 101.2 98.8) (width 1) (layer B.Cu) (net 1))
 (via (at 101.1 98.9) (size 1.6) (drill 0.6) (layers F.Cu B.Cu) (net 1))
 (segment (start 139 101.75) (end 139 98.8) (width 1.5) (layer F.Cu) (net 1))
 (via (at 139 98.8) (size 1.6) (drill 0.6) (layers F.Cu B.Cu) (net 1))
 (segment (start 139.04 105) (end 139.04 101.79) (width 2) (layer F.Cu) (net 1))
 (segment (start 139.04 101.79) (end 139 101.75) (width 2) (layer F.Cu) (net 1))
 (segment (start 106.00228 105.6) (end 107.7 105.6) (width 0.8) (layer F.Cu) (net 12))
 (segment (start 107.7 105.6) (end 108 105.3) (width 0.8) (layer F.Cu) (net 12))
 (segment (start 129.7 103.5824) (end 131.38 101.9024) (width 0.6) (layer F.Cu) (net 9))
 (segment (start 131.38 101.9024) (end 131.38 101.75) (width 0.6) (layer F.Cu) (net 9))
 (segment (start 129.7 104.65) (end 129.7 103.5824) (width 0.6) (layer F.Cu) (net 9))
 (segment (start 127.8 106.4) (end 127.95 106.4) (width 0.6) (layer F.Cu) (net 9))
 (segment (start 127.95 106.4) (end 129.7 104.65) (width 0.6) (layer F.Cu) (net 9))
 (segment (start 127 107.4) (end 129.1724 107.4) (width 0.4) (layer F.Cu) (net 10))
 (segment (start 129.1724 107.4) (end 131.42 105.1524) (width 0.4) (layer F.Cu) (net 10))
 (segment (start 131.42 105.1524) (end 131.42 105) (width 0.4) (layer F.Cu) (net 10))
 (segment (start 126.7 107.1) (end 127 107.4) (width 0.4) (layer F.Cu) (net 10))
 (segment (start 126.7 105.55) (end 126.7 107.1) (width 0.4) (layer F.Cu) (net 10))
 (segment (start 127.65 104.6) (end 126.7 105.55) (width 0.4) (layer F.Cu) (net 10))
 (segment (start 125.6 102.9) (end 125.95 102.9) (width 0.6) (layer F.Cu) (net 10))
 (segment (start 125.95 102.9) (end 127.65 104.6) (width 0.6) (layer F.Cu) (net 10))
 (segment (start 127.65 104.6) (end 127.8 104.6) (width 0.6) (layer F.Cu) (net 10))
 (segment (start 103 104.65) (end 103 103.3) (width 0.6) (layer F.Cu) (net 11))
 (segment (start 103 104.65) (end 101.45 104.65) (width 0.8) (layer F.Cu) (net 11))
 (segment (start 101.45 104.65) (end 101 104.2) (width 0.8) (layer F.Cu) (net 11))
 (segment (start 108 102.76) (end 108 100.1) (width 1) (layer F.Cu) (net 2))
 (segment (start 108 100.1) (end 108.1 100) (width 1) (layer F.Cu) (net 2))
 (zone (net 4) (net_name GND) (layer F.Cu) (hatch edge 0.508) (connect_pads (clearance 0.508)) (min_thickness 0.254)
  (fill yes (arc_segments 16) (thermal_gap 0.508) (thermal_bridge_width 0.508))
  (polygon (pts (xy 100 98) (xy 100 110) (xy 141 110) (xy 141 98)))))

